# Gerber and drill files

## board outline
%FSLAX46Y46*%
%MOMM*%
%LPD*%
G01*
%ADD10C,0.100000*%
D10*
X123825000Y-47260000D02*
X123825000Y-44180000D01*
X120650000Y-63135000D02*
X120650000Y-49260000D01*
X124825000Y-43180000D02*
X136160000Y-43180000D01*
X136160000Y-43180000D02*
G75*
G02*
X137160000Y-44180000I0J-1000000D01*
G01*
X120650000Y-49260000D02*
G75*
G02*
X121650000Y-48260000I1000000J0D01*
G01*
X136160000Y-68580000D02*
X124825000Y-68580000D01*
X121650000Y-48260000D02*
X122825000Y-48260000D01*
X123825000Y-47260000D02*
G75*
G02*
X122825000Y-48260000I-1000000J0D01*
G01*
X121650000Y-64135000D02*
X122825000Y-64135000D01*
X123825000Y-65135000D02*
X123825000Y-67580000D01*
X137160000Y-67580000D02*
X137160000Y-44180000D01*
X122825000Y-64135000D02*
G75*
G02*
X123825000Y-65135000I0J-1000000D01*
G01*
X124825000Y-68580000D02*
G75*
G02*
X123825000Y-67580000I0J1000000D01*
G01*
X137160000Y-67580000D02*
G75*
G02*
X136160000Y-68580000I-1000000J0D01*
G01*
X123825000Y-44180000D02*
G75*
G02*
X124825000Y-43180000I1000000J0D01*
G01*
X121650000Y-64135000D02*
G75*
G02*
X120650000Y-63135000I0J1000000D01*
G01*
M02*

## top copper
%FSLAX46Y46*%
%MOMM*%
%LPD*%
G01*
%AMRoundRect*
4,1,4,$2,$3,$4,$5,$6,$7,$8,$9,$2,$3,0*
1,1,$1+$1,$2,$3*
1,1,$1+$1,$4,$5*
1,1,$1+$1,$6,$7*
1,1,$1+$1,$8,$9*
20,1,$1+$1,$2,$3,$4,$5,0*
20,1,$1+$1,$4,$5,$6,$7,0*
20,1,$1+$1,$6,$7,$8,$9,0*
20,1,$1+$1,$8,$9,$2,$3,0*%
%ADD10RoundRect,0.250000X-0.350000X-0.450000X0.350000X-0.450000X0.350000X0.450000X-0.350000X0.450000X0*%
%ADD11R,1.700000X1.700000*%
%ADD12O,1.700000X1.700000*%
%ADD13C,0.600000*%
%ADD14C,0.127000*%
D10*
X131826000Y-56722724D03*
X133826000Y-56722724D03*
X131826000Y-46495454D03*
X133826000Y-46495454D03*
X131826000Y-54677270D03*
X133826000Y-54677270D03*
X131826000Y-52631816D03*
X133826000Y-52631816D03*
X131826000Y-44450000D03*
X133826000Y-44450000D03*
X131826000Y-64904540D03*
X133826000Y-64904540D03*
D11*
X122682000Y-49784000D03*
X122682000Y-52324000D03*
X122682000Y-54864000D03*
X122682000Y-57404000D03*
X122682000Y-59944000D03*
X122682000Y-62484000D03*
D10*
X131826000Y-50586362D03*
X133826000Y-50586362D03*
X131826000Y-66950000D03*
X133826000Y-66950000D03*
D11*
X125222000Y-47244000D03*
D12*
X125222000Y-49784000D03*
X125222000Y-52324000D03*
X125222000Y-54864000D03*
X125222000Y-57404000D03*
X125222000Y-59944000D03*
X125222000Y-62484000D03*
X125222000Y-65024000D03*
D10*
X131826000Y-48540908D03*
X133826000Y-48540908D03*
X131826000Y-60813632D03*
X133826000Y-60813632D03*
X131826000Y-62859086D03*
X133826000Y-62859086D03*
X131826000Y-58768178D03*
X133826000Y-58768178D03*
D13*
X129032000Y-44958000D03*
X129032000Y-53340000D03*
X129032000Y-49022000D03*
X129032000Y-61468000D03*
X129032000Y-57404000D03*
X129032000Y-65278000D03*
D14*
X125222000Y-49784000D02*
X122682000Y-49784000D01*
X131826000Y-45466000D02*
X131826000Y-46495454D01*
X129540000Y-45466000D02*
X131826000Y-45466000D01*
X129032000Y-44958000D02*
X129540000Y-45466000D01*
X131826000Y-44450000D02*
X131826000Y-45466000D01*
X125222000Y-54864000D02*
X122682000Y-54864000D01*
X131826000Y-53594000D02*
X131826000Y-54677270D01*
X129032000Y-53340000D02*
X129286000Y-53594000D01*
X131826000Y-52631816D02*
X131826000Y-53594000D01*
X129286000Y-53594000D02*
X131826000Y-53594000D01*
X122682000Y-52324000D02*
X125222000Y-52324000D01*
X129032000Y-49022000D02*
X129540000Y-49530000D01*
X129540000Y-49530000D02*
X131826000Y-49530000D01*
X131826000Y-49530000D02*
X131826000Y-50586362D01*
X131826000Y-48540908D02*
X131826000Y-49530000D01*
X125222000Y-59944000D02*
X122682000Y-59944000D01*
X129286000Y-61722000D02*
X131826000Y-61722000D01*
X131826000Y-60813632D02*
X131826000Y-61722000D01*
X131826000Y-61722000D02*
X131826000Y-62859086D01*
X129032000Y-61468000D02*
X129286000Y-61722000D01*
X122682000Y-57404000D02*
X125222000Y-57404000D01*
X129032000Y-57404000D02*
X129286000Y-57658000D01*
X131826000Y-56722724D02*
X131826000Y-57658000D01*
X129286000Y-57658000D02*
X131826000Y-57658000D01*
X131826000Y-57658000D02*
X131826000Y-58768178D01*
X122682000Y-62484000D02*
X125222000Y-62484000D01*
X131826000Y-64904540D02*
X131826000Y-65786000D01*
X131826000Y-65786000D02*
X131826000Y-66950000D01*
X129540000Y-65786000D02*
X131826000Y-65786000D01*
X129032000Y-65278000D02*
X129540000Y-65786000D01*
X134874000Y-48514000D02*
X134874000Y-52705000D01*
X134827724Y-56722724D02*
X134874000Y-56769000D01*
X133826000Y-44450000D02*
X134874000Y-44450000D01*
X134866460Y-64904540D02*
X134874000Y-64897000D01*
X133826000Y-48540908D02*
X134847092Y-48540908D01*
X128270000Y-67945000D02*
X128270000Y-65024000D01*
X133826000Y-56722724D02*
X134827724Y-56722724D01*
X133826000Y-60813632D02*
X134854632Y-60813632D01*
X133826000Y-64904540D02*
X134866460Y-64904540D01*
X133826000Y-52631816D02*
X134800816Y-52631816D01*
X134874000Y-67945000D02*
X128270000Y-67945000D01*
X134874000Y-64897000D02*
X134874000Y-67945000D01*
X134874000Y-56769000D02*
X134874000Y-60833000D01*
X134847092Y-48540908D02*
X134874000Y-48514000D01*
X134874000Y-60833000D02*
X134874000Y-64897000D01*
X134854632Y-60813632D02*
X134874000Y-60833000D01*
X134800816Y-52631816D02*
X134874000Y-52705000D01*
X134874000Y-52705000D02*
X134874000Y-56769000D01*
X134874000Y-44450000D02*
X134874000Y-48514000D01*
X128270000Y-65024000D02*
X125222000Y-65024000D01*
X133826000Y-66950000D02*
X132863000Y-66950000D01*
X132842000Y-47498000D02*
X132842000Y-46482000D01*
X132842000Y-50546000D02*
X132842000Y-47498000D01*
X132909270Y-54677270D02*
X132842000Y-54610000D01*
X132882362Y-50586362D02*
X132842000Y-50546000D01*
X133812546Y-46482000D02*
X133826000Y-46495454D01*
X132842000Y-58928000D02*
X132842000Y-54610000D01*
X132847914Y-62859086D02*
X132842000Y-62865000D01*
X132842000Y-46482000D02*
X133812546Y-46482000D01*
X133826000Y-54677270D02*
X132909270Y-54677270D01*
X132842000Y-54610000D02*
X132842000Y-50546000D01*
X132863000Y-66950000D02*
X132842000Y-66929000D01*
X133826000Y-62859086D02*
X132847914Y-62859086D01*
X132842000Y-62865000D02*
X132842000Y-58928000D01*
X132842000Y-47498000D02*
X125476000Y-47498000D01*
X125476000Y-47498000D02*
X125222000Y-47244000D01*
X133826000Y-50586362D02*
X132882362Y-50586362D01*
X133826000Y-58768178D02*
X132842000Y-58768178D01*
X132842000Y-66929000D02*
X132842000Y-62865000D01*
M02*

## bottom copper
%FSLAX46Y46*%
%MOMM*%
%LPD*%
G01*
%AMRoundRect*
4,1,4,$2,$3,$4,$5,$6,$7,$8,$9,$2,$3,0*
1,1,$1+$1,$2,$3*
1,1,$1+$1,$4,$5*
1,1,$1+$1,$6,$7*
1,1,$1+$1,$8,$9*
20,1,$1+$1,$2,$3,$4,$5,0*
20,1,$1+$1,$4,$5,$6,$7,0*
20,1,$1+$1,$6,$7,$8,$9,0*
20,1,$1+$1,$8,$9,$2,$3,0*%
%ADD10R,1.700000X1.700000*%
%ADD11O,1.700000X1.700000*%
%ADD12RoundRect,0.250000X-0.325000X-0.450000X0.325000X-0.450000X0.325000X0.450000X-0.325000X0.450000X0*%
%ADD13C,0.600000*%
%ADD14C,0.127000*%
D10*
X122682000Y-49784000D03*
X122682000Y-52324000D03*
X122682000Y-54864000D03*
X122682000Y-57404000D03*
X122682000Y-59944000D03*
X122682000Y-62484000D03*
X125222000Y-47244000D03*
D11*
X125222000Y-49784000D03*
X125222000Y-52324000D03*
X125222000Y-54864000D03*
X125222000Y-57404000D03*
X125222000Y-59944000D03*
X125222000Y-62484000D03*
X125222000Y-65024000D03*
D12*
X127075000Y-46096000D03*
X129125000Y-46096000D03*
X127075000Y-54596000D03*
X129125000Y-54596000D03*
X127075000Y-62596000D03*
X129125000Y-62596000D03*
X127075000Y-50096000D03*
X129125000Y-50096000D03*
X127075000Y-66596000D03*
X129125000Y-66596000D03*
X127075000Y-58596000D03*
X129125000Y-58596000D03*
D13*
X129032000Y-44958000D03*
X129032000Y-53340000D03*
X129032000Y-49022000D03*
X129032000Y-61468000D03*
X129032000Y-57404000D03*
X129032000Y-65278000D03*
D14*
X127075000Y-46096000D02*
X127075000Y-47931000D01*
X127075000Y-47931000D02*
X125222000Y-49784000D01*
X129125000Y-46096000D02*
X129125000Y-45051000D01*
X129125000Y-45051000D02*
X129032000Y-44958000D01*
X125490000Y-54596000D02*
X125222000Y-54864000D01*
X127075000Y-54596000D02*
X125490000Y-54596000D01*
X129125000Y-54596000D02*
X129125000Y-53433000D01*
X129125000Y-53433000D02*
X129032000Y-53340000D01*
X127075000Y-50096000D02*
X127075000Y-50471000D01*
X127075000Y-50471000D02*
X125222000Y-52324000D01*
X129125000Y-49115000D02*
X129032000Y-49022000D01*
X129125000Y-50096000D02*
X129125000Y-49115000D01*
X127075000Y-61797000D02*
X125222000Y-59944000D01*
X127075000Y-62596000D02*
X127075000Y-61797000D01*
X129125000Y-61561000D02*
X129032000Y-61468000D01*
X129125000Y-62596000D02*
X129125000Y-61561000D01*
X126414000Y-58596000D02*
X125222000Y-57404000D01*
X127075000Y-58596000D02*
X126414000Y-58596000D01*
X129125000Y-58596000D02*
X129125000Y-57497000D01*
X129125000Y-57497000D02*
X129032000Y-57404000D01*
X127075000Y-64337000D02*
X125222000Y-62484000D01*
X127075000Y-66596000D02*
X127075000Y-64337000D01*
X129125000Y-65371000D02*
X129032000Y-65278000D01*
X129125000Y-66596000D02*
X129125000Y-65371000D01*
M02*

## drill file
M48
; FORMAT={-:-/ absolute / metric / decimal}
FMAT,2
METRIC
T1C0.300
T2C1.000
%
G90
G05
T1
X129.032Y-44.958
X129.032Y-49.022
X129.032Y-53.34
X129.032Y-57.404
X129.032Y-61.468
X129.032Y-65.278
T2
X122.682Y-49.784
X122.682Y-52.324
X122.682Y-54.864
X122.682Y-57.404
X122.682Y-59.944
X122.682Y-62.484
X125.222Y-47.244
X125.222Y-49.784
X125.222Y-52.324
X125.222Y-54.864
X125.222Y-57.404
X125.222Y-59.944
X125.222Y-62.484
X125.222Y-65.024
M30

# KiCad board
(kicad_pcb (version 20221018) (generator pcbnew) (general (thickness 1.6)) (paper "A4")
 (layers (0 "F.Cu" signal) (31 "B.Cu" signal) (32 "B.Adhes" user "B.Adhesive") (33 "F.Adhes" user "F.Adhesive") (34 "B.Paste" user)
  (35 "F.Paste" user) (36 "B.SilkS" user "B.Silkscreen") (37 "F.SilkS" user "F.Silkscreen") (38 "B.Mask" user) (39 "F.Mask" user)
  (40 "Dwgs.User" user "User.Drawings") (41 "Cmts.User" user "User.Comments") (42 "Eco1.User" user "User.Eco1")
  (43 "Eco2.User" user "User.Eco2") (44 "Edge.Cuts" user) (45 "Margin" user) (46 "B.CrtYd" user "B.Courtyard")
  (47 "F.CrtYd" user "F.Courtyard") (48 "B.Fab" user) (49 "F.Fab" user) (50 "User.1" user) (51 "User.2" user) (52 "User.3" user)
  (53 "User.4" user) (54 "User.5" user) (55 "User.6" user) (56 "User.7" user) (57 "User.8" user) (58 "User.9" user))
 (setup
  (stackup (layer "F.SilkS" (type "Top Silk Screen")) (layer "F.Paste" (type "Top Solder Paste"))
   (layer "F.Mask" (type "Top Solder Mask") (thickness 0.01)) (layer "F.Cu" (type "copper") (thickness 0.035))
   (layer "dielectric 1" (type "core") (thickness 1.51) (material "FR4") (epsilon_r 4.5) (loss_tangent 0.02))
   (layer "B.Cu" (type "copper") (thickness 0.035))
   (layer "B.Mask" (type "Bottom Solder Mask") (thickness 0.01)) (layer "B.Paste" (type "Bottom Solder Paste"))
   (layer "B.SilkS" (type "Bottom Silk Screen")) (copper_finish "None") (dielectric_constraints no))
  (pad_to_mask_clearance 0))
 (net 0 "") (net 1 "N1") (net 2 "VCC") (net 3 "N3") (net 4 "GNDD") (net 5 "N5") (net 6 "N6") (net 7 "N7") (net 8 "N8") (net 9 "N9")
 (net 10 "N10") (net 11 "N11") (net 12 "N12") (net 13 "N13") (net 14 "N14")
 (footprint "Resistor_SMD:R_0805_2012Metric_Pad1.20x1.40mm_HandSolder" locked (layer "F.Cu") (at 132.826 56.722724)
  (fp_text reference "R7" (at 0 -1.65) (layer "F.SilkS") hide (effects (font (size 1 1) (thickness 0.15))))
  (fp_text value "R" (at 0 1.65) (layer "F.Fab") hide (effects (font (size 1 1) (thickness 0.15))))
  (pad "1" smd roundrect locked (at -1 0) (size 1.2 1.4) (layers "F.Cu" "F.Paste" "F.Mask") (roundrect_rratio 0.2083333333) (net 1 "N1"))
  (pad "2" smd roundrect locked (at 1 0) (size 1.2 1.4) (layers "F.Cu" "F.Paste" "F.Mask") (roundrect_rratio 0.2083333333) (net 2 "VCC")))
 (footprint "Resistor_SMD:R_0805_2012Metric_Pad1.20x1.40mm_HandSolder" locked (layer "F.Cu") (at 132.826 46.495454)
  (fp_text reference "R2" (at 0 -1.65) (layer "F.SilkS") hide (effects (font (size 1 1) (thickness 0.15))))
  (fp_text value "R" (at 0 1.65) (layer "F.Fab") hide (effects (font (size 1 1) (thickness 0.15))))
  (pad "1" smd roundrect locked (at -1 0) (size 1.2 1.4) (layers "F.Cu" "F.Paste" "F.Mask") (roundrect_rratio 0.2083333333) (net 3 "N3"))
  (pad "2" smd roundrect locked (at 1 0) (size 1.2 1.4) (layers "F.Cu" "F.Paste" "F.Mask") (roundrect_rratio 0.2083333333) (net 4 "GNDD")))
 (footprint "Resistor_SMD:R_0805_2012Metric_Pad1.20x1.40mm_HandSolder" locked (layer "F.Cu") (at 132.826 54.67727)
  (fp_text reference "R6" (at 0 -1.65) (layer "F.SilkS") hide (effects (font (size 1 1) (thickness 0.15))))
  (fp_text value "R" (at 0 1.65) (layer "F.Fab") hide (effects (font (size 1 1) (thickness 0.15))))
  (pad "1" smd roundrect locked (at -1 0) (size 1.2 1.4) (layers "F.Cu" "F.Paste" "F.Mask") (roundrect_rratio 0.2083333333) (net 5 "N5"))
  (pad "2" smd roundrect locked (at 1 0) (size 1.2 1.4) (layers "F.Cu" "F.Paste" "F.Mask") (roundrect_rratio 0.2083333333) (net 4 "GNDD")))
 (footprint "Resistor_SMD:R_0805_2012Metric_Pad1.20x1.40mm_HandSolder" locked (layer "F.Cu") (at 132.826 52.631816)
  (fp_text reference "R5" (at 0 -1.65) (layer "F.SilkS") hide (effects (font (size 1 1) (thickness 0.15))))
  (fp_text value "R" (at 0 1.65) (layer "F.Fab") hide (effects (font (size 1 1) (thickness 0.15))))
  (pad "1" smd roundrect locked (at -1 0) (size 1.2 1.4) (layers "F.Cu" "F.Paste" "F.Mask") (roundrect_rratio 0.2083333333) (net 5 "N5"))
  (pad "2" smd roundrect locked (at 1 0) (size 1.2 1.4) (layers "F.Cu" "F.Paste" "F.Mask") (roundrect_rratio 0.2083333333) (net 2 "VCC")))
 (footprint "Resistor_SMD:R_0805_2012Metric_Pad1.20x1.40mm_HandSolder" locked (layer "F.Cu") (at 132.826 44.45)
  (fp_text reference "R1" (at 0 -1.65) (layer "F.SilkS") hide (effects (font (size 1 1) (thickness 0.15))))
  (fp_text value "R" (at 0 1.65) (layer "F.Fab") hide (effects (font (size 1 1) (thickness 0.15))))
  (pad "1" smd roundrect locked (at -1 0) (size 1.2 1.4) (layers "F.Cu" "F.Paste" "F.Mask") (roundrect_rratio 0.2083333333) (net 3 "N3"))
  (pad "2" smd roundrect locked (at 1 0) (size 1.2 1.4) (layers "F.Cu" "F.Paste" "F.Mask") (roundrect_rratio 0.2083333333) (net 2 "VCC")))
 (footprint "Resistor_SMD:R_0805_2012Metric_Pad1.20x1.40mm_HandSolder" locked (layer "F.Cu") (at 132.826 64.90454)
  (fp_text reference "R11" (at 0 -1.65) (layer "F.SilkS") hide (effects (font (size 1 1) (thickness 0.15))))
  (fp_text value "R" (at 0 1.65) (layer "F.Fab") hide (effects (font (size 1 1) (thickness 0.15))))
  (pad "1" smd roundrect locked (at -1 0) (size 1.2 1.4) (layers "F.Cu" "F.Paste" "F.Mask") (roundrect_rratio 0.2083333333) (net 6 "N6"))
  (pad "2" smd roundrect locked (at 1 0) (size 1.2 1.4) (layers "F.Cu" "F.Paste" "F.Mask") (roundrect_rratio 0.2083333333) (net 2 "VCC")))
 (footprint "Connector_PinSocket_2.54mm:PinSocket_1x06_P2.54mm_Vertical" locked (layer "F.Cu") (at 122.682 49.784)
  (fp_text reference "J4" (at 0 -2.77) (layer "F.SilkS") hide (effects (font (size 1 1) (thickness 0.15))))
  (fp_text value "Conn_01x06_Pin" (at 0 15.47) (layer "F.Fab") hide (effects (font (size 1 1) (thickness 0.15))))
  (pad "1" thru_hole rect locked (at 0 0) (size 1.7 1.7) (drill 1) (layers "*.Cu" "*.Mask") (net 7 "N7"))
  (pad "2" thru_hole rect locked (at 0 2.54) (size 1.7 1.7) (drill 1) (layers "*.Cu" "*.Mask") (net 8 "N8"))
  (pad "3" thru_hole rect locked (at 0 5.08) (size 1.7 1.7) (drill 1) (layers "*.Cu" "*.Mask") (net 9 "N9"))
  (pad "4" thru_hole rect locked (at 0 7.62) (size 1.7 1.7) (drill 1) (layers "*.Cu" "*.Mask") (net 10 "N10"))
  (pad "5" thru_hole rect locked (at 0 10.16) (size 1.7 1.7) (drill 1) (layers "*.Cu" "*.Mask") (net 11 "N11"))
  (pad "6" thru_hole rect locked (at 0 12.7) (size 1.7 1.7) (drill 1) (layers "*.Cu" "*.Mask") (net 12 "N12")))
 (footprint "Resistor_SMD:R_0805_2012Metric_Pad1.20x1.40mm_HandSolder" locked (layer "F.Cu") (at 132.826 50.586362)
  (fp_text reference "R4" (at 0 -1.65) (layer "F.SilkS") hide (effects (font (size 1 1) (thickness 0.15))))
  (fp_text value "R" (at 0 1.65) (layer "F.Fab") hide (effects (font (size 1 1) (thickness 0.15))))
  (pad "1" smd roundrect locked (at -1 0) (size 1.2 1.4) (layers "F.Cu" "F.Paste" "F.Mask") (roundrect_rratio 0.2083333333) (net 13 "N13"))
  (pad "2" smd roundrect locked (at 1 0) (size 1.2 1.4) (layers "F.Cu" "F.Paste" "F.Mask") (roundrect_rratio 0.2083333333) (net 4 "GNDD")))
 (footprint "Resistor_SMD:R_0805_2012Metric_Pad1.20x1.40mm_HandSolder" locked (layer "F.Cu") (at 132.826 66.95)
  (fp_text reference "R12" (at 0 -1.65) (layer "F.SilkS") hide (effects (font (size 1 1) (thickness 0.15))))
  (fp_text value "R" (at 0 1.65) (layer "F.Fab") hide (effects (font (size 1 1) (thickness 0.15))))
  (pad "1" smd roundrect locked (at -1 0) (size 1.2 1.4) (layers "F.Cu" "F.Paste" "F.Mask") (roundrect_rratio 0.2083333333) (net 6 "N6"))
  (pad "2" smd roundrect locked (at 1 0) (size 1.2 1.4) (layers "F.Cu" "F.Paste" "F.Mask") (roundrect_rratio 0.2083333333) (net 4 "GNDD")))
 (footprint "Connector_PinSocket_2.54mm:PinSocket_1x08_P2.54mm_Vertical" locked (layer "F.Cu") (at 125.222 47.244)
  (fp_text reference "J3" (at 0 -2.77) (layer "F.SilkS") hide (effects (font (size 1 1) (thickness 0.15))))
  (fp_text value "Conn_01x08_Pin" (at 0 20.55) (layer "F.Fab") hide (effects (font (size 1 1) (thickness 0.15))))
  (pad "1" thru_hole rect locked (at 0 0) (size 1.7 1.7) (drill 1) (layers "*.Cu" "*.Mask") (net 4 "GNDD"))
  (pad "2" thru_hole oval locked (at 0 2.54) (size 1.7 1.7) (drill 1) (layers "*.Cu" "*.Mask") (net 7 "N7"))
  (pad "3" thru_hole oval locked (at 0 5.08) (size 1.7 1.7) (drill 1) (layers "*.Cu" "*.Mask") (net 8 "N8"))
  (pad "4" thru_hole oval locked (at 0 7.62) (size 1.7 1.7) (drill 1) (layers "*.Cu" "*.Mask") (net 9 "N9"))
  (pad "5" thru_hole oval locked (at 0 10.16) (size 1.7 1.7) (drill 1) (layers "*.Cu" "*.Mask") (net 10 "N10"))
  (pad "6" thru_hole oval locked (at 0 12.7) (size 1.7 1.7) (drill 1) (layers "*.Cu" "*.Mask") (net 11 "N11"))
  (pad "7" thru_hole oval locked (at 0 15.24) (size 1.7 1.7) (drill 1) (layers "*.Cu" "*.Mask") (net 12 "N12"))
  (pad "8" thru_hole oval locked (at 0 17.78) (size 1.7 1.7) (drill 1) (layers "*.Cu" "*.Mask") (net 2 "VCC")))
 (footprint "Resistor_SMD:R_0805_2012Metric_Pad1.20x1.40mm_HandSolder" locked (layer "F.Cu") (at 132.826 48.540908)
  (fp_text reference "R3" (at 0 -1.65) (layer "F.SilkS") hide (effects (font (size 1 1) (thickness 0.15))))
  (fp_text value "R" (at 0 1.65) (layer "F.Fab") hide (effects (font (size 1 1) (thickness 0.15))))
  (pad "1" smd roundrect locked (at -1 0) (size 1.2 1.4) (layers "F.Cu" "F.Paste" "F.Mask") (roundrect_rratio 0.2083333333) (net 13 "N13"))
  (pad "2" smd roundrect locked (at 1 0) (size 1.2 1.4) (layers "F.Cu" "F.Paste" "F.Mask") (roundrect_rratio 0.2083333333) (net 2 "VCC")))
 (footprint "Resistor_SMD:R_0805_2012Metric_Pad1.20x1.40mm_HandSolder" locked (layer "F.Cu") (at 132.826 60.813632)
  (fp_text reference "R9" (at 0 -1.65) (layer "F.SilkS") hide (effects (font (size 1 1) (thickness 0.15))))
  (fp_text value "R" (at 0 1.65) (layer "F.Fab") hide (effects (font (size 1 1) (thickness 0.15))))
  (pad "1" smd roundrect locked (at -1 0) (size 1.2 1.4) (layers "F.Cu" "F.Paste" "F.Mask") (roundrect_rratio 0.2083333333) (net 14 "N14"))
  (pad "2" smd roundrect locked (at 1 0) (size 1.2 1.4) (layers "F.Cu" "F.Paste" "F.Mask") (roundrect_rratio 0.2083333333) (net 2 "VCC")))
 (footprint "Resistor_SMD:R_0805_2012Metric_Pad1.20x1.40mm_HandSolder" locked (layer "F.Cu") (at 132.826 62.859086)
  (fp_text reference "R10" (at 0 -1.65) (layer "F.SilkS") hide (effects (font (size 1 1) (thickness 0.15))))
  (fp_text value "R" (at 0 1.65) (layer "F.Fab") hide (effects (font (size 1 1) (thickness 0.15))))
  (pad "1" smd roundrect locked (at -1 0) (size 1.2 1.4) (layers "F.Cu" "F.Paste" "F.Mask") (roundrect_rratio 0.2083333333) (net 14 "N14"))
  (pad "2" smd roundrect locked (at 1 0) (size 1.2 1.4) (layers "F.Cu" "F.Paste" "F.Mask") (roundrect_rratio 0.2083333333) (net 4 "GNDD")))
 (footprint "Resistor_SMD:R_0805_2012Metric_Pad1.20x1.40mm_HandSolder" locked (layer "F.Cu") (at 132.826 58.768178)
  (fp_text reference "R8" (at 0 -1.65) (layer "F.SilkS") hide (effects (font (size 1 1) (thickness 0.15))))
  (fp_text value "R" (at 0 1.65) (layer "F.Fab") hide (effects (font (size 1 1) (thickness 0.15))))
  (pad "1" smd roundrect locked (at -1 0) (size 1.2 1.4) (layers "F.Cu" "F.Paste" "F.Mask") (roundrect_rratio 0.2083333333) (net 1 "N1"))
  (pad "2" smd roundrect locked (at 1 0) (size 1.2 1.4) (layers "F.Cu" "F.Paste" "F.Mask") (roundrect_rratio 0.2083333333) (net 4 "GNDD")))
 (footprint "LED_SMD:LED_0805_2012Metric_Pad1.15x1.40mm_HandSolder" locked (layer "B.Cu") (at 128.1 46.096)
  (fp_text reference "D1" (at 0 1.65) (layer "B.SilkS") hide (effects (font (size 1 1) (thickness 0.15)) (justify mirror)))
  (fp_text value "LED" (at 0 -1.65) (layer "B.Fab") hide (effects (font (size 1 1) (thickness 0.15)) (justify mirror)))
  (pad "1" smd roundrect locked (at -1.025 0) (size 1.15 1.4) (layers "B.Cu" "B.Paste" "B.Mask") (roundrect_rratio 0.2173913043)
   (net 7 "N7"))
  (pad "2" smd roundrect locked (at 1.025 0) (size 1.15 1.4) (layers "B.Cu" "B.Paste" "B.Mask") (roundrect_rratio 0.2173913043) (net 3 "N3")))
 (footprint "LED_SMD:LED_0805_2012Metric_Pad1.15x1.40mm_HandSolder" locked (layer "B.Cu") (at 128.1 54.596)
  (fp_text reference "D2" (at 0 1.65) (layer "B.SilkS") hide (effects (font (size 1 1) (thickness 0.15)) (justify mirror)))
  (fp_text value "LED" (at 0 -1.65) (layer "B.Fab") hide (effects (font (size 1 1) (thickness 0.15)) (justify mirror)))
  (pad "1" smd roundrect locked (at -1.025 0) (size 1.15 1.4) (layers "B.Cu" "B.Paste" "B.Mask") (roundrect_rratio 0.2173913043)
   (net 9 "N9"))
  (pad "2" smd roundrect locked (at 1.025 0) (size 1.15 1.4) (layers "B.Cu" "B.Paste" "B.Mask") (roundrect_rratio 0.2173913043) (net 5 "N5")))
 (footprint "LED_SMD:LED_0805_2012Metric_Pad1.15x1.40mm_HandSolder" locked (layer "B.Cu") (at 128.1 62.596)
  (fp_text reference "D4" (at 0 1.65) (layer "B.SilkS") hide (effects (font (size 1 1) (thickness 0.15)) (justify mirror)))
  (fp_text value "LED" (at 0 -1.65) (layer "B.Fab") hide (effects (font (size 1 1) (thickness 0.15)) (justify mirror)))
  (pad "1" smd roundrect locked (at -1.025 0) (size 1.15 1.4) (layers "B.Cu" "B.Paste" "B.Mask") (roundrect_rratio 0.2173913043)
   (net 11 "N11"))
  (pad "2" smd roundrect locked (at 1.025 0) (size 1.15 1.4) (layers "B.Cu" "B.Paste" "B.Mask") (roundrect_rratio 0.2173913043)
   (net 14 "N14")))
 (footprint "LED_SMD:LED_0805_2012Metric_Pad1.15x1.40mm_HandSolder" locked (layer "B.Cu") (at 128.1 50.096)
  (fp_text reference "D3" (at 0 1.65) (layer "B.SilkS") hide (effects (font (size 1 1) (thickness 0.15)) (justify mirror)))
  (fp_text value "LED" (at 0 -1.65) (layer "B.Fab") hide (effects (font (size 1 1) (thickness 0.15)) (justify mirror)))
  (pad "1" smd roundrect locked (at -1.025 0) (size 1.15 1.4) (layers "B.Cu" "B.Paste" "B.Mask") (roundrect_rratio 0.2173913043)
   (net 8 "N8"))
  (pad "2" smd roundrect locked (at 1.025 0) (size 1.15 1.4) (layers "B.Cu" "B.Paste" "B.Mask") (roundrect_rratio 0.2173913043)
   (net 13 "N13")))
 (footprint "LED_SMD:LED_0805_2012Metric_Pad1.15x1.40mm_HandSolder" (layer "B.Cu") (at 128.1 66.596)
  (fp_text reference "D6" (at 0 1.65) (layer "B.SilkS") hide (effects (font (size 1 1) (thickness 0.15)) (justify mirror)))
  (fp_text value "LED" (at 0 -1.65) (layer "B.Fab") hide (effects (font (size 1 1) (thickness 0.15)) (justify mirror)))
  (pad "1" smd roundrect (at -1.025 0) (size 1.15 1.4) (layers "B.Cu" "B.Paste" "B.Mask") (roundrect_rratio 0.2173913043) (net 12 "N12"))
  (pad "2" smd roundrect (at 1.025 0) (size 1.15 1.4) (layers "B.Cu" "B.Paste" "B.Mask") (roundrect_rratio 0.2173913043) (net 6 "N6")))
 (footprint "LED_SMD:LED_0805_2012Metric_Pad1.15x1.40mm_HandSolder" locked (layer "B.Cu") (at 128.1 58.596)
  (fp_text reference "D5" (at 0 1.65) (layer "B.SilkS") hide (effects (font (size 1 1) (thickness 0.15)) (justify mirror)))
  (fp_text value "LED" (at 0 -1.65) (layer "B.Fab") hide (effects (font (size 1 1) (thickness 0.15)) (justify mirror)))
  (pad "1" smd roundrect locked (at -1.025 0) (size 1.15 1.4) (layers "B.Cu" "B.Paste" "B.Mask") (roundrect_rratio 0.2173913043)
   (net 10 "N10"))
  (pad "2" smd roundrect locked (at 1.025 0) (size 1.15 1.4) (layers "B.Cu" "B.Paste" "B.Mask") (roundrect_rratio 0.2173913043) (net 1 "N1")))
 (gr_line (start 123.825 47.26) (end 123.825 44.18) (stroke (width 0.1) (type default)) (layer "Edge.Cuts"))
 (gr_line (start 120.65 63.135) (end 120.65 49.26) (stroke (width 0.1) (type default)) (layer "Edge.Cuts"))
 (gr_line (start 124.825 43.18) (end 136.16 43.18) (stroke (width 0.1) (type default)) (layer "Edge.Cuts"))
 (gr_arc (start 136.16 43.18) (mid 136.867107 43.472893) (end 137.16 44.18) (stroke (width 0.1) (type default)) (layer "Edge.Cuts"))
 (gr_arc (start 120.65 49.26) (mid 120.942893 48.552893) (end 121.65 48.26) (stroke (width 0.1) (type default)) (layer "Edge.Cuts"))
 (gr_line (start 136.16 68.58) (end 124.825 68.58) (stroke (width 0.1) (type default)) (layer "Edge.Cuts"))
 (gr_line (start 121.65 48.26) (end 122.825 48.26) (stroke (width 0.1) (type default)) (layer "Edge.Cuts"))
 (gr_arc (start 123.825 47.26) (mid 123.532107 47.967107) (end 122.825 48.26) (stroke (width 0.1) (type default)) (layer "Edge.Cuts"))
 (gr_line (start 121.65 64.135) (end 122.825 64.135) (stroke (width 0.1) (type default)) (layer "Edge.Cuts"))
 (gr_line (start 123.825 65.135) (end 123.825 67.58) (stroke (width 0.1) (type default)) (layer "Edge.Cuts"))
 (gr_line (start 137.16 67.58) (end 137.16 44.18) (stroke (width 0.1) (type default)) (layer "Edge.Cuts"))
 (gr_arc (start 122.825 64.135) (mid 123.532107 64.427893) (end 123.825 65.135) (stroke (width 0.1) (type default)) (layer "Edge.Cuts"))
 (gr_arc (start 124.825 68.58) (mid 124.117893 68.287107) (end 123.825 67.58) (stroke (width 0.1) (type default)) (layer "Edge.Cuts"))
 (gr_arc (start 137.16 67.58) (mid 136.867107 68.287107) (end 136.16 68.58) (stroke (width 0.1) (type default)) (layer "Edge.Cuts"))
 (gr_arc (start 123.825 44.18) (mid 124.117893 43.472893) (end 124.825 43.18) (stroke (width 0.1) (type default)) (layer "Edge.Cuts"))
 (gr_arc (start 121.65 64.135) (mid 120.942893 63.842107) (end 120.65 63.135) (stroke (width 0.1) (type default)) (layer "Edge.Cuts"))
 (segment (start 125.222 49.784) (end 122.682 49.784) (width 0.127) (layer "F.Cu") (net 7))
 (segment (start 127.075 46.096) (end 127.075 47.931) (width 0.127) (layer "B.Cu") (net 7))
 (segment (start 127.075 47.931) (end 125.222 49.784) (width 0.127) (layer "B.Cu") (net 7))
 (segment (start 131.826 45.466) (end 131.826 46.495454) (width 0.127) (layer "F.Cu") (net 3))
 (segment (start 129.54 45.466) (end 131.826 45.466) (width 0.127) (layer "F.Cu") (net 3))
 (segment (start 129.032 44.958) (end 129.54 45.466) (width 0.127) (layer "F.Cu") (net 3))
 (segment (start 131.826 44.45) (end 131.826 45.466) (width 0.127) (layer "F.Cu") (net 3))
 (via (at 129.032 44.958) (size 0.6) (drill 0.3) (layers "F.Cu" "B.Cu") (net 3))
 (segment (start 129.125 46.096) (end 129.125 45.051) (width 0.127) (layer "B.Cu") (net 3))
 (segment (start 129.125 45.051) (end 129.032 44.958) (width 0.127) (layer "B.Cu") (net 3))
 (segment (start 125.222 54.864) (end 122.682 54.864) (width 0.127) (layer "F.Cu") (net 9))
 (segment (start 125.49 54.596) (end 125.222 54.864) (width 0.127) (layer "B.Cu") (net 9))
 (segment (start 127.075 54.596) (end 125.49 54.596) (width 0.127) (layer "B.Cu") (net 9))
 (segment (start 131.826 53.594) (end 131.826 54.67727) (width 0.127) (layer "F.Cu") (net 5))
 (segment (start 129.032 53.34) (end 129.286 53.594) (width 0.127) (layer "F.Cu") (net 5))
 (segment (start 131.826 52.631816) (end 131.826 53.594) (width 0.127) (layer "F.Cu") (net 5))
 (segment (start 129.286 53.594) (end 131.826 53.594) (width 0.127) (layer "F.Cu") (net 5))
 (via (at 129.032 53.34) (size 0.6) (drill 0.3) (layers "F.Cu" "B.Cu") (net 5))
 (segment (start 129.125 54.596) (end 129.125 53.433) (width 0.127) (layer "B.Cu") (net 5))
 (segment (start 129.125 53.433) (end 129.032 53.34) (width 0.127) (layer "B.Cu") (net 5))
 (segment (start 122.682 52.324) (end 125.222 52.324) (width 0.127) (layer "F.Cu") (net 8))
 (segment (start 127.075 50.096) (end 127.075 50.471) (width 0.127) (layer "B.Cu") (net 8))
 (segment (start 127.075 50.471) (end 125.222 52.324) (width 0.127) (layer "B.Cu") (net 8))
 (segment (start 129.032 49.022) (end 129.54 49.53) (width 0.127) (layer "F.Cu") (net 13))
 (segment (start 129.54 49.53) (end 131.826 49.53) (width 0.127) (layer "F.Cu") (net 13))
 (segment (start 131.826 49.53) (end 131.826 50.586362) (width 0.127) (layer "F.Cu") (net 13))
 (segment (start 131.826 48.540908) (end 131.826 49.53) (width 0.127) (layer "F.Cu") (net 13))
 (via (at 129.032 49.022) (size 0.6) (drill 0.3) (layers "F.Cu" "B.Cu") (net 13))
 (segment (start 129.125 49.115) (end 129.032 49.022) (width 0.127) (layer "B.Cu") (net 13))
 (segment (start 129.125 50.096) (end 129.125 49.115) (width 0.127) (layer "B.Cu") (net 13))
 (segment (start 125.222 59.944) (end 122.682 59.944) (width 0.127) (layer "F.Cu") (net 11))
 (segment (start 127.075 61.797) (end 125.222 59.944) (width 0.127) (layer "B.Cu") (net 11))
 (segment (start 127.075 62.596) (end 127.075 61.797) (width 0.127) (layer "B.Cu") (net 11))
 (segment (start 129.286 61.722) (end 131.826 61.722) (width 0.127) (layer "F.Cu") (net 14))
 (segment (start 131.826 60.813632) (end 131.826 61.722) (width 0.127) (layer "F.Cu") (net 14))
 (segment (start 131.826 61.722) (end 131.826 62.859086) (width 0.127) (layer "F.Cu") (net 14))
 (segment (start 129.032 61.468) (end 129.286 61.722) (width 0.127) (layer "F.Cu") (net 14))
 (via (at 129.032 61.468) (size 0.6) (drill 0.3) (layers "F.Cu" "B.Cu") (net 14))
 (segment (start 129.125 61.561) (end 129.032 61.468) (width 0.127) (layer "B.Cu") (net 14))
 (segment (start 129.125 62.596) (end 129.125 61.561) (width 0.127) (layer "B.Cu") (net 14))
 (segment (start 122.682 57.404) (end 125.222 57.404) (width 0.127) (layer "F.Cu") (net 10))
 (segment (start 126.414 58.596) (end 125.222 57.404) (width 0.127) (layer "B.Cu") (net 10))
 (segment (start 127.075 58.596) (end 126.414 58.596) (width 0.127) (layer "B.Cu") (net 10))
 (segment (start 129.032 57.404) (end 129.286 57.658) (width 0.127) (layer "F.Cu") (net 1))
 (segment (start 131.826 56.722724) (end 131.826 57.658) (width 0.127) (layer "F.Cu") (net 1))
 (segment (start 129.286 57.658) (end 131.826 57.658) (width 0.127) (layer "F.Cu") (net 1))
 (segment (start 131.826 57.658) (end 131.826 58.768178) (width 0.127) (layer "F.Cu") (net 1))
 (via (at 129.032 57.404) (size 0.6) (drill 0.3) (layers "F.Cu" "B.Cu") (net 1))
 (segment (start 129.125 58.596) (end 129.125 57.497) (width 0.127) (layer "B.Cu") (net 1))
 (segment (start 129.125 57.497) (end 129.032 57.404) (width 0.127) (layer "B.Cu") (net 1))
 (segment (start 122.682 62.484) (end 125.222 62.484) (width 0.127) (layer "F.Cu") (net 12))
 (segment (start 127.075 64.337) (end 125.222 62.484) (width 0.127) (layer "B.Cu") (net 12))
 (segment (start 127.075 66.596) (end 127.075 64.337) (width 0.127) (layer "B.Cu") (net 12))
 (segment (start 131.826 64.90454) (end 131.826 65.786) (width 0.127) (layer "F.Cu") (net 6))
 (segment (start 131.826 65.786) (end 131.826 66.95) (width 0.127) (layer "F.Cu") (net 6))
 (segment (start 129.54 65.786) (end 131.826 65.786) (width 0.127) (layer "F.Cu") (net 6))
 (segment (start 129.032 65.278) (end 129.54 65.786) (width 0.127) (layer "F.Cu") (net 6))
 (via (at 129.032 65.278) (size 0.6) (drill 0.3) (layers "F.Cu" "B.Cu") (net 6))
 (segment (start 129.125 65.371) (end 129.032 65.278) (width 0.127) (layer "B.Cu") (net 6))
 (segment (start 129.125 66.596) (end 129.125 65.371) (width 0.127) (layer "B.Cu") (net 6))
 (segment (start 134.874 48.514) (end 134.874 52.705) (width 0.127) (layer "F.Cu") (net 2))
 (segment (start 134.827724 56.722724) (end 134.874 56.769) (width 0.127) (layer "F.Cu") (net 2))
 (segment (start 133.826 44.45) (end 134.874 44.45) (width 0.127) (layer "F.Cu") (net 2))
 (segment (start 134.86646 64.90454) (end 134.874 64.897) (width 0.127) (layer "F.Cu") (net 2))
 (segment (start 133.826 48.540908) (end 134.847092 48.540908) (width 0.127) (layer "F.Cu") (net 2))
 (segment (start 128.27 67.945) (end 128.27 65.024) (width 0.127) (layer "F.Cu") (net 2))
 (segment (start 133.826 56.722724) (end 134.827724 56.722724) (width 0.127) (layer "F.Cu") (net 2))
 (segment (start 133.826 60.813632) (end 134.854632 60.813632) (width 0.127) (layer "F.Cu") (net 2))
 (segment (start 133.826 64.90454) (end 134.86646 64.90454) (width 0.127) (layer "F.Cu") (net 2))
 (segment (start 133.826 52.631816) (end 134.800816 52.631816) (width 0.127) (layer "F.Cu") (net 2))
 (segment (start 134.874 67.945) (end 128.27 67.945) (width 0.127) (layer "F.Cu") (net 2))
 (segment (start 134.874 64.897) (end 134.874 67.945) (width 0.127) (layer "F.Cu") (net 2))
 (segment (start 134.874 56.769) (end 134.874 60.833) (width 0.127) (layer "F.Cu") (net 2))
 (segment (start 134.847092 48.540908) (end 134.874 48.514) (width 0.127) (layer "F.Cu") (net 2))
 (segment (start 134.874 60.833) (end 134.874 64.897) (width 0.127) (layer "F.Cu") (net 2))
 (segment (start 134.854632 60.813632) (end 134.874 60.833) (width 0.127) (layer "F.Cu") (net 2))
 (segment (start 134.800816 52.631816) (end 134.874 52.705) (width 0.127) (layer "F.Cu") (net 2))
 (segment (start 134.874 52.705) (end 134.874 56.769) (width 0.127) (layer "F.Cu") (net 2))
 (segment (start 134.874 44.45) (end 134.874 48.514) (width 0.127) (layer "F.Cu") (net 2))
 (segment (start 128.27 65.024) (end 125.222 65.024) (width 0.127) (layer "F.Cu") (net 2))
 (segment (start 133.826 66.95) (end 132.863 66.95) (width 0.127) (layer "F.Cu") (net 4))
 (segment (start 132.842 47.498) (end 132.842 46.482) (width 0.127) (layer "F.Cu") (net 4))
 (segment (start 132.842 50.546) (end 132.842 47.498) (width 0.127) (layer "F.Cu") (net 4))
 (segment (start 132.90927 54.67727) (end 132.842 54.61) (width 0.127) (layer "F.Cu") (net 4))
 (segment (start 132.882362 50.586362) (end 132.842 50.546) (width 0.127) (layer "F.Cu") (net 4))
 (segment (start 133.812546 46.482) (end 133.826 46.495454) (width 0.127) (layer "F.Cu") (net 4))
 (segment (start 132.842 58.928) (end 132.842 54.61) (width 0.127) (layer "F.Cu") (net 4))
 (segment (start 132.847914 62.859086) (end 132.842 62.865) (width 0.127) (layer "F.Cu") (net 4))
 (segment (start 132.842 46.482) (end 133.812546 46.482) (width 0.127) (layer "F.Cu") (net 4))
 (segment (start 133.826 54.67727) (end 132.90927 54.67727) (width 0.127) (layer "F.Cu") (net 4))
 (segment (start 132.842 54.61) (end 132.842 50.546) (width 0.127) (layer "F.Cu") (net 4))
 (segment (start 132.863 66.95) (end 132.842 66.929) (width 0.127) (layer "F.Cu") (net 4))
 (segment (start 133.826 62.859086) (end 132.847914 62.859086) (width 0.127) (layer "F.Cu") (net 4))
 (segment (start 132.842 62.865) (end 132.842 58.928) (width 0.127) (layer "F.Cu") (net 4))
 (segment (start 132.842 47.498) (end 125.476 47.498) (width 0.127) (layer "F.Cu") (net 4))
 (segment (start 125.476 47.498) (end 125.222 47.244) (width 0.127) (layer "F.Cu") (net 4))
 (segment (start 133.826 50.586362) (end 132.882362 50.586362) (width 0.127) (layer "F.Cu") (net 4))
 (segment (start 133.826 58.768178) (end 132.842 58.768178) (width 0.127) (layer "F.Cu") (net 4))
 (segment (start 132.842 66.929) (end 132.842 62.865) (width 0.127) (layer "F.Cu") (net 4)))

